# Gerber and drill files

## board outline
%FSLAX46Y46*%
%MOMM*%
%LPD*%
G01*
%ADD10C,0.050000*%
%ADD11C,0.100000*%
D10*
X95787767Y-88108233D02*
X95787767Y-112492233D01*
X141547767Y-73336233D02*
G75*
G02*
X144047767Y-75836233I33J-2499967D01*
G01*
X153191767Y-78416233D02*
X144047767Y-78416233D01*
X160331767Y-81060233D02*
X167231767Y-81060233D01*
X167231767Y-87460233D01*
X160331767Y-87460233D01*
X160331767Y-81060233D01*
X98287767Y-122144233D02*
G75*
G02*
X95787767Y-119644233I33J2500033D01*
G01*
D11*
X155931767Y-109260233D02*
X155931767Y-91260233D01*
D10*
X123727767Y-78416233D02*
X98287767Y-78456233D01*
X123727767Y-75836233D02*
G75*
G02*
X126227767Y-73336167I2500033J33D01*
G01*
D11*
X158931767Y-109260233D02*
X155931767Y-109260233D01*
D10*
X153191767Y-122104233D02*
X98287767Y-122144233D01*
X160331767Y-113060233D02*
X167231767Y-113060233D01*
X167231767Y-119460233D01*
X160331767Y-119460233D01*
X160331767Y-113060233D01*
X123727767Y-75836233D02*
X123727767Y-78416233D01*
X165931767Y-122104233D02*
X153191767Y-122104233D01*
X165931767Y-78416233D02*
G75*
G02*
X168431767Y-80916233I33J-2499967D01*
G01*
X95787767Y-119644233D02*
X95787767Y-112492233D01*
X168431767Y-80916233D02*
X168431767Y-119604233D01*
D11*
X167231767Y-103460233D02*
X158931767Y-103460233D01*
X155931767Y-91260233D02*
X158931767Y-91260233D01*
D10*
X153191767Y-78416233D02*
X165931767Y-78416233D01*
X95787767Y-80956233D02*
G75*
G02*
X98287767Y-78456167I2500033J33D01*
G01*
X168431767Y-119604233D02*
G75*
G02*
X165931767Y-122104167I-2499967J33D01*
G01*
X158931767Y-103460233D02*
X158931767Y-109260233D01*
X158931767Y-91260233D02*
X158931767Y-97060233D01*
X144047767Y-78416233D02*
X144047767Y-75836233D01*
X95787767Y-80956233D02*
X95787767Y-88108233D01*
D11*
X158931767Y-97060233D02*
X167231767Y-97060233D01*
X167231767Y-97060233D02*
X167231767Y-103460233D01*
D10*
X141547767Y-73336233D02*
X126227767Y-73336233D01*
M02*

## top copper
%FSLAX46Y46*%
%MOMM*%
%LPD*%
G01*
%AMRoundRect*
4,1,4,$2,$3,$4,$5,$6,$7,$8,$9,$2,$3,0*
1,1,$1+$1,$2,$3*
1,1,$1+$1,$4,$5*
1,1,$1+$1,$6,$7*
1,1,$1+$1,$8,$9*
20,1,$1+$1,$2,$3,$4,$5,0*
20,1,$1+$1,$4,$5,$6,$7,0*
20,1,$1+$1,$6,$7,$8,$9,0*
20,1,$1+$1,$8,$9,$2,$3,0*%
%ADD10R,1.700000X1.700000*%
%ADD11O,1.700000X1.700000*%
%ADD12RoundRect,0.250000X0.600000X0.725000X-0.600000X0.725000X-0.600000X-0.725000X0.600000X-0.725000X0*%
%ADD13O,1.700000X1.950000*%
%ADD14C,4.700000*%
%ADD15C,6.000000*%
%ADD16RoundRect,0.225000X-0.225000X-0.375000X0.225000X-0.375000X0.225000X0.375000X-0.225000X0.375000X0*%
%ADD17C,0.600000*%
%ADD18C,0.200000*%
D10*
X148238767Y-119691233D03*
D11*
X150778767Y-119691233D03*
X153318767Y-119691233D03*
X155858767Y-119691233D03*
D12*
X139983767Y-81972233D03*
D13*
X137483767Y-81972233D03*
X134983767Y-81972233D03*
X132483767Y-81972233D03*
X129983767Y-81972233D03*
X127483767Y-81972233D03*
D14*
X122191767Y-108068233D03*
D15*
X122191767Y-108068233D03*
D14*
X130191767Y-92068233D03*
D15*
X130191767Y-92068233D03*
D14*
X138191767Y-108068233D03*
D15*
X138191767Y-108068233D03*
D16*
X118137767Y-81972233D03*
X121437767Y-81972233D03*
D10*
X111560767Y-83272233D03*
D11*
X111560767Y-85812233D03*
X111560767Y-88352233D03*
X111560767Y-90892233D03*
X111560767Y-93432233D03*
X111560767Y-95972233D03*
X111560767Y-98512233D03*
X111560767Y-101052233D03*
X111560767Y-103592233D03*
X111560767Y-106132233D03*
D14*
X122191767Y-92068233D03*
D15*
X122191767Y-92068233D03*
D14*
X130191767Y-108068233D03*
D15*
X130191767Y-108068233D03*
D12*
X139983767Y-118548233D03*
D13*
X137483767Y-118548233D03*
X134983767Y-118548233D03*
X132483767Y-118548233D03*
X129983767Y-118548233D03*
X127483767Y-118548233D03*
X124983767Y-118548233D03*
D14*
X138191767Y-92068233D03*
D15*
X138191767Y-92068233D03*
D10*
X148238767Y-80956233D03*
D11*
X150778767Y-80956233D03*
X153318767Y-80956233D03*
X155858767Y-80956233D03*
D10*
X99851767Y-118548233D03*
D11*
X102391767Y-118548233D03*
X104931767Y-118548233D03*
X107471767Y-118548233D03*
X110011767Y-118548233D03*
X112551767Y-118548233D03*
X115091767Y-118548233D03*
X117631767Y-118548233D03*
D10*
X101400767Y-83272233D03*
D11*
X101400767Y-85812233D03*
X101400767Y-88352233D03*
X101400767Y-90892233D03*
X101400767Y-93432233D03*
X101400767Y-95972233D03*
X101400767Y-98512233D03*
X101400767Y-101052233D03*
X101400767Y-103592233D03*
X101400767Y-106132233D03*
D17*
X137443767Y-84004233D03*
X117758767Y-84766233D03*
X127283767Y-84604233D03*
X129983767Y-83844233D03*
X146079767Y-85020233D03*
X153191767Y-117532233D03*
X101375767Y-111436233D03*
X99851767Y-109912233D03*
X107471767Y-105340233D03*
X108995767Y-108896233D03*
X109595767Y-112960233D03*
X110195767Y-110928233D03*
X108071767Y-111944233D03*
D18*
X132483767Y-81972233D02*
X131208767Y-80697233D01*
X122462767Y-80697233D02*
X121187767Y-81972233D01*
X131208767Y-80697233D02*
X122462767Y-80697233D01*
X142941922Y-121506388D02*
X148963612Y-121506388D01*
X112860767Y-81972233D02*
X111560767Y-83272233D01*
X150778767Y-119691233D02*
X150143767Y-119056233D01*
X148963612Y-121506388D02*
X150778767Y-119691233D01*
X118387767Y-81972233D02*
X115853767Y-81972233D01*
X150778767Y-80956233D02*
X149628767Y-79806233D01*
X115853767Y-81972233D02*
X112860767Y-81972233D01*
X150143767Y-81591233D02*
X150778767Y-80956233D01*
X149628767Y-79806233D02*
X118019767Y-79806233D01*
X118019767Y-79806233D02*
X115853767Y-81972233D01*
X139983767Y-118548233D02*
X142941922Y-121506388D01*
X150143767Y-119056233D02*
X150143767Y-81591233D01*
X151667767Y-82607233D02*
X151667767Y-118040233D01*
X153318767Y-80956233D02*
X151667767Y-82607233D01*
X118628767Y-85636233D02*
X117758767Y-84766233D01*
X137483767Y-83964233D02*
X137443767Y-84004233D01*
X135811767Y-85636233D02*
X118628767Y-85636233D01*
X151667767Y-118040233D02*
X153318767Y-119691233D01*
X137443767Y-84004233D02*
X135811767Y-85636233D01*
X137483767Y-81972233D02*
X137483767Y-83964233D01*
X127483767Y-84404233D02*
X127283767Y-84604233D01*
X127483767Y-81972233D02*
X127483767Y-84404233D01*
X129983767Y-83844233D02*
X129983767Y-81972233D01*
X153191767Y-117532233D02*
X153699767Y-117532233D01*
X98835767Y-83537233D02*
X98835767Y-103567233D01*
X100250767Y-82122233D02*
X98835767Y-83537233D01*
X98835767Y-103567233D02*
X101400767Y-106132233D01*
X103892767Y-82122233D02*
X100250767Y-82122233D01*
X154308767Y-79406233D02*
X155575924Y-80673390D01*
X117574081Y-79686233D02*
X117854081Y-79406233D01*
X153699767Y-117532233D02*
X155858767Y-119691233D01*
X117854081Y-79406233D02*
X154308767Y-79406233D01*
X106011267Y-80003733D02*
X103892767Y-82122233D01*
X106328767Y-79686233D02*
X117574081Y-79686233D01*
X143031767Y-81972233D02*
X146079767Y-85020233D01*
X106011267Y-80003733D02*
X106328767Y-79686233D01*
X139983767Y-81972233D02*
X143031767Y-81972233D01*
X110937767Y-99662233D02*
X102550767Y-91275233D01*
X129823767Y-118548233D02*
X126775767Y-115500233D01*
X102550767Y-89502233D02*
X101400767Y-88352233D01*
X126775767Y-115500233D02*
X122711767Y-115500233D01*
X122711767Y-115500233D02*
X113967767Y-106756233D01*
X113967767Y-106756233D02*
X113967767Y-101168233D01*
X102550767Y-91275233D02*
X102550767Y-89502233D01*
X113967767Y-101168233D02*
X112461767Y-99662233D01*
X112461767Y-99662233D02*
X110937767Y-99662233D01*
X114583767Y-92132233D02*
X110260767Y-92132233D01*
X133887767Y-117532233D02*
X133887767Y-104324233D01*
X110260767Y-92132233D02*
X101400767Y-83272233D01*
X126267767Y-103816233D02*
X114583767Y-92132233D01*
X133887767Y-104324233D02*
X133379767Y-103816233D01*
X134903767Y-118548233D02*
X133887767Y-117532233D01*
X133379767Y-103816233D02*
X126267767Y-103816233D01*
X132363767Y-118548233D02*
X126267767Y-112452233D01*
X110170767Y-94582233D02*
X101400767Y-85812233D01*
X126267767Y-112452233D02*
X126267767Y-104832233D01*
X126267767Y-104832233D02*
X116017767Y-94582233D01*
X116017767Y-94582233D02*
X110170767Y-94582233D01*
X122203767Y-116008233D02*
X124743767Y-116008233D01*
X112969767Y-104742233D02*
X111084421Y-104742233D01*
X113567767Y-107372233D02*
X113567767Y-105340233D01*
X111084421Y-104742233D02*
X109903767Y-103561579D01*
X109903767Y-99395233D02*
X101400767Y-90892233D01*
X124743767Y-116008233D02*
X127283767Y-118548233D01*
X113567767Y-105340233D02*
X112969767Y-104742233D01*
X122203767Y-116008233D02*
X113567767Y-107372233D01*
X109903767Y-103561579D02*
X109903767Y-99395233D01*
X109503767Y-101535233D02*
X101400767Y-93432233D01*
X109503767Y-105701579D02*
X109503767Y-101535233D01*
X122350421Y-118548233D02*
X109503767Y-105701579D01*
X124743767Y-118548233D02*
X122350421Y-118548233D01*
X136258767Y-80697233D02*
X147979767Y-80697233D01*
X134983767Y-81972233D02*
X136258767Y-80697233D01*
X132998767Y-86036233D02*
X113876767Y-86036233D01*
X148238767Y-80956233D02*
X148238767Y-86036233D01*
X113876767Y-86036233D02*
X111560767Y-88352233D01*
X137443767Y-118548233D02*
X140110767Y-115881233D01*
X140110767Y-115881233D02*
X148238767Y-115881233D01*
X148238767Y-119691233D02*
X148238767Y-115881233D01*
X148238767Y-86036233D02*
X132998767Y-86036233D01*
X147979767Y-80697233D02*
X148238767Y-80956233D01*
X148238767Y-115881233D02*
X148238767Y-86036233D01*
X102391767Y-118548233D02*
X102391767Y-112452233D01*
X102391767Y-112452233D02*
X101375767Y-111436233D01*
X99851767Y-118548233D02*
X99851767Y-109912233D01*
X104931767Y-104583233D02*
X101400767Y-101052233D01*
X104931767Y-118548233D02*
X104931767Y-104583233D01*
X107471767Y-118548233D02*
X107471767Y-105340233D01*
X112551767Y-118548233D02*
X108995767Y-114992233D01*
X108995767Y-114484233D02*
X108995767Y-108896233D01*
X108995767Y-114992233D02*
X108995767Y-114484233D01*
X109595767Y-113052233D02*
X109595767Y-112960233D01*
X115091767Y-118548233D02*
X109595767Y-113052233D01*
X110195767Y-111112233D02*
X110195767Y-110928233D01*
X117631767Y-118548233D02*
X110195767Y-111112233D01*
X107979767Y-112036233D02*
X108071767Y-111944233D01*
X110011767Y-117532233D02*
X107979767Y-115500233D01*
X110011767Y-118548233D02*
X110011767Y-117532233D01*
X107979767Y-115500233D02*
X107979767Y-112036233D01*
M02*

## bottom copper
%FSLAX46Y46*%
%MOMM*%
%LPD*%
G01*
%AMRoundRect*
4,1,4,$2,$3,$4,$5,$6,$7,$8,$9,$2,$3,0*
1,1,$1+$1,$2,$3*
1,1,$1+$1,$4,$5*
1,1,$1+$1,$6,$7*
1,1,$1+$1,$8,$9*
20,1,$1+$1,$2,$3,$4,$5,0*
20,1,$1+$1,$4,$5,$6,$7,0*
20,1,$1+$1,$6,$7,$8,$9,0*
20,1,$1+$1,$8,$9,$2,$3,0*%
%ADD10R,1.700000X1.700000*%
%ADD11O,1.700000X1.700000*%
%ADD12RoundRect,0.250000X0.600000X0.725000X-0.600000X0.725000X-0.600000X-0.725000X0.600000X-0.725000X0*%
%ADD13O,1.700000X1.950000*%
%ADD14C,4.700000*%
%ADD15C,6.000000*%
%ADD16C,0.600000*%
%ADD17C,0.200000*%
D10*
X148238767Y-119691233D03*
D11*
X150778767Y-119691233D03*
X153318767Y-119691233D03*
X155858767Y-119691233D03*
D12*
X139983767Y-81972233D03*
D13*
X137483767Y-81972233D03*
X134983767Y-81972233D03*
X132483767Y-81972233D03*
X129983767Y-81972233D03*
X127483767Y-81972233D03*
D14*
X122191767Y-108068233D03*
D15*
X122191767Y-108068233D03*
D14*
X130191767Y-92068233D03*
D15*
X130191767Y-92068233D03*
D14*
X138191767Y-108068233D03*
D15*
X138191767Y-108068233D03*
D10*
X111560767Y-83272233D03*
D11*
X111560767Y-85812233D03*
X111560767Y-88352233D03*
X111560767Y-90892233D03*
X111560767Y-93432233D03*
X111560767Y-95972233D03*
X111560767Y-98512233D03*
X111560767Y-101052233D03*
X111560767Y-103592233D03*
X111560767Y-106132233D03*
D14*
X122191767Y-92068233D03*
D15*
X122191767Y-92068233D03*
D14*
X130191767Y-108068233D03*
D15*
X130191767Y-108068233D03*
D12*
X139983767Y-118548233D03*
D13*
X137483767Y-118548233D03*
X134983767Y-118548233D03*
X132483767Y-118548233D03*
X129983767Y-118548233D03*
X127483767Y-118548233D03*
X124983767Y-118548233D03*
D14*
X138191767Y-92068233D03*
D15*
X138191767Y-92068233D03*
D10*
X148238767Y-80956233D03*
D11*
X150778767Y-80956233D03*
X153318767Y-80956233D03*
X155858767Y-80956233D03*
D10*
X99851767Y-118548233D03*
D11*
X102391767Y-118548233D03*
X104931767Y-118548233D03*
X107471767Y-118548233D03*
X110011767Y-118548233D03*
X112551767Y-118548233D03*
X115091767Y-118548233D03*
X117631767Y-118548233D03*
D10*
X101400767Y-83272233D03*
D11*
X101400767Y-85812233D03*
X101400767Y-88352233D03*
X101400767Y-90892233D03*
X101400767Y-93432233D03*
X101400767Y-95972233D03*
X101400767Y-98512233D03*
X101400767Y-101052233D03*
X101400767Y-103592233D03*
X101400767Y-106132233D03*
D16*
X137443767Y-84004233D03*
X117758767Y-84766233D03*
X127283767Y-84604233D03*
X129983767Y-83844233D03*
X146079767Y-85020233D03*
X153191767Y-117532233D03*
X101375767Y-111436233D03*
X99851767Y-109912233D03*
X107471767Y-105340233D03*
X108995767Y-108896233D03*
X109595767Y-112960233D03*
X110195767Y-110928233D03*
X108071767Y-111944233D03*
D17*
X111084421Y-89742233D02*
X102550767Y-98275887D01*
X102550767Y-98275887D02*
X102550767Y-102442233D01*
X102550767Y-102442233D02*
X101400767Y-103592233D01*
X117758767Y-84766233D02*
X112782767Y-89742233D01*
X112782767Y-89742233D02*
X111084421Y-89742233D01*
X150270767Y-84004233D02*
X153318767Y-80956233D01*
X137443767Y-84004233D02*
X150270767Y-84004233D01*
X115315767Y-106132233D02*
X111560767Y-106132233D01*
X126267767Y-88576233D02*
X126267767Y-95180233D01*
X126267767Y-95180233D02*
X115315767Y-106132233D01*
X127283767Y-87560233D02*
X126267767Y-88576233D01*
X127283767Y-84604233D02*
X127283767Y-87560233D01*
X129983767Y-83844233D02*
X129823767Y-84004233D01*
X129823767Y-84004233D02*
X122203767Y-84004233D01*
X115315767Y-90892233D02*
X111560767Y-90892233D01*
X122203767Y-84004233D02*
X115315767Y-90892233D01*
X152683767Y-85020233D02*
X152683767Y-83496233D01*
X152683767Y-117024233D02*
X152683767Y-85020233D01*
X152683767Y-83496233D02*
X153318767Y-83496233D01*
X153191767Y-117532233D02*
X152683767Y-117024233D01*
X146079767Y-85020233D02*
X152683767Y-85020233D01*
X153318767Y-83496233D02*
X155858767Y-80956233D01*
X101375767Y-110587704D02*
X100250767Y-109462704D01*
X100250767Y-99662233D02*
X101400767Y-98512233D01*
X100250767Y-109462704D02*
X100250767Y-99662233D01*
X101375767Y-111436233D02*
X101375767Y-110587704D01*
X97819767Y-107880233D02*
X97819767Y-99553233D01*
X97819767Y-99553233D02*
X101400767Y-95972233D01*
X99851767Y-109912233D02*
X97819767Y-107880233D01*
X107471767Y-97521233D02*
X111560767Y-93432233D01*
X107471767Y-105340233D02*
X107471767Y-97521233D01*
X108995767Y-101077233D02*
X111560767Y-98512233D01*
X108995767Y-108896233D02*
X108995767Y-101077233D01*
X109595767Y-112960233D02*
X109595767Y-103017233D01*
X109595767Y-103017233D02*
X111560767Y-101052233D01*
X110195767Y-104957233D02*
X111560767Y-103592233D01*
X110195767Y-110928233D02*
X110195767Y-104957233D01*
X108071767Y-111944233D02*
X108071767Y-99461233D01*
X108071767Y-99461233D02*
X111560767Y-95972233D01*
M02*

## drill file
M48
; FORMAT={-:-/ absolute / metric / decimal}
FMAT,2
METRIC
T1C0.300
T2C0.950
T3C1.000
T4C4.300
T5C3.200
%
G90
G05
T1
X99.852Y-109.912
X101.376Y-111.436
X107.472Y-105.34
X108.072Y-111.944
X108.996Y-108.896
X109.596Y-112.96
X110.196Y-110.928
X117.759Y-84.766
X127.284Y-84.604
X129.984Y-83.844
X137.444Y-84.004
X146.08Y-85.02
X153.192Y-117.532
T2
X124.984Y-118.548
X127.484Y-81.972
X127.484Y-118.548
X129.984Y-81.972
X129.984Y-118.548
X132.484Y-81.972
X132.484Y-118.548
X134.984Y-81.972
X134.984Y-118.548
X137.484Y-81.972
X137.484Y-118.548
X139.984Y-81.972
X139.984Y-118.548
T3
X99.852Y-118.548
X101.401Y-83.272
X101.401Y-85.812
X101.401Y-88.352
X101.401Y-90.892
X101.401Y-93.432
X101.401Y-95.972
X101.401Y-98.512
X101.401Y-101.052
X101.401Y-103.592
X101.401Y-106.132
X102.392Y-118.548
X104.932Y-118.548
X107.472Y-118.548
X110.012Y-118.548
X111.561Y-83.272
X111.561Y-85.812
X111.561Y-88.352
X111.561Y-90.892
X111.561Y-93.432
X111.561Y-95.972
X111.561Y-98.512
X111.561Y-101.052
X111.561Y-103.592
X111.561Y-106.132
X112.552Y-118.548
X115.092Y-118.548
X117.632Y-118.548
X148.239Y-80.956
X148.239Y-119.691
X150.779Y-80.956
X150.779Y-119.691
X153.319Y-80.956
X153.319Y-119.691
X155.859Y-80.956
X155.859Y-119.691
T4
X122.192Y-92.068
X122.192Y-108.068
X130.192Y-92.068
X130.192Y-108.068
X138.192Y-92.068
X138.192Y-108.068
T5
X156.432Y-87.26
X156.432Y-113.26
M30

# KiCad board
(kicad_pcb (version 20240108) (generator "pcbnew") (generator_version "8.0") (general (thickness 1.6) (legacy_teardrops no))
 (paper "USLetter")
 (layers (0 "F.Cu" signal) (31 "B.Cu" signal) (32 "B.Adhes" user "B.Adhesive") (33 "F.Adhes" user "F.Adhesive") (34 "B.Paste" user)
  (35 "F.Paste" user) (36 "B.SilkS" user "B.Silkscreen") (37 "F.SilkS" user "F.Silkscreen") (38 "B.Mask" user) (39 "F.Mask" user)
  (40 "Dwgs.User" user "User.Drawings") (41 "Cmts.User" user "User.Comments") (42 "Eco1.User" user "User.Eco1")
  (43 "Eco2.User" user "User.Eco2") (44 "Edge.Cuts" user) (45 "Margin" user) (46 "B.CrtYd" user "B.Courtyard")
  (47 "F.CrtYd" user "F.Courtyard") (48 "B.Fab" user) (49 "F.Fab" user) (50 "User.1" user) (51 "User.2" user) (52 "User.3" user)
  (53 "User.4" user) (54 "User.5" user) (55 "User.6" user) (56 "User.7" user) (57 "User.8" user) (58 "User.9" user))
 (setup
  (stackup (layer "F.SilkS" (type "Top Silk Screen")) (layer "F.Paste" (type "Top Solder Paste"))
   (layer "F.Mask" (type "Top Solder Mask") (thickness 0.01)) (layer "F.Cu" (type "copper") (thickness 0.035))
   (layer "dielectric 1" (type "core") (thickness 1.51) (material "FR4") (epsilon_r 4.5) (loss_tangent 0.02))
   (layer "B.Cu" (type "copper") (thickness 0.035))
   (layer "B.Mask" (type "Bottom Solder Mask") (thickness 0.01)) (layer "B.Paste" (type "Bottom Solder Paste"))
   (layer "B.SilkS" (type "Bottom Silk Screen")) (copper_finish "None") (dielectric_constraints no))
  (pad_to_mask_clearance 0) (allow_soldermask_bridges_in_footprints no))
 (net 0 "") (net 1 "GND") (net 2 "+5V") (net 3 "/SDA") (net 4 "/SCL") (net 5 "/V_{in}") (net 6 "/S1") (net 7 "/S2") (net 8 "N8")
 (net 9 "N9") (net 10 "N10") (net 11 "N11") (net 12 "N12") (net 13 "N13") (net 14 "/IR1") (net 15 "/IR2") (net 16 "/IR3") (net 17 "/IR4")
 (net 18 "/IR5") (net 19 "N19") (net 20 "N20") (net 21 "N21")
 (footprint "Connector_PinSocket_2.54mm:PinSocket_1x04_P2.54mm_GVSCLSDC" (layer "F.Cu") (at 148.238767 119.691233 90)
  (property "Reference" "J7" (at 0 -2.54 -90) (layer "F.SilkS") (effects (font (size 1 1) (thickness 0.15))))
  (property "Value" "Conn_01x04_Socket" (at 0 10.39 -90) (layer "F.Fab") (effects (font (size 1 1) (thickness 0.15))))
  (pad "1" thru_hole rect (at 0 0 90) (size 1.7 1.7) (drill 1) (layers "*.Cu" "*.Mask") (remove_unused_layers no) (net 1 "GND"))
  (pad "2" thru_hole oval (at 0 2.54 90) (size 1.7 1.7) (drill 1) (layers "*.Cu" "*.Mask") (remove_unused_layers no) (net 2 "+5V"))
  (pad "3" thru_hole oval (at 0 5.08 90) (size 1.7 1.7) (drill 1) (layers "*.Cu" "*.Mask") (remove_unused_layers no) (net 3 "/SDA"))
  (pad "4" thru_hole oval (at 0 7.62 90) (size 1.7 1.7) (drill 1) (layers "*.Cu" "*.Mask") (remove_unused_layers no) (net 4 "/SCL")))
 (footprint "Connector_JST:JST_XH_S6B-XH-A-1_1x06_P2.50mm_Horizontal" (layer "F.Cu") (at 139.983767 81.972233 180)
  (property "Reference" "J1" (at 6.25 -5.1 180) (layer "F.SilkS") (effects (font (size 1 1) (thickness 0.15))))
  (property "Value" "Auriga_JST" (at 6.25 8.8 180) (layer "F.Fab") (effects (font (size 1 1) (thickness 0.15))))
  (pad "1" thru_hole roundrect (at 0 0 180) (size 1.7 1.95) (drill 0.95) (layers "*.Cu" "*.Mask") (remove_unused_layers no)
   (roundrect_rratio 0.147059) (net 4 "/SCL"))
  (pad "2" thru_hole oval (at 2.5 0 180) (size 1.7 1.95) (drill 0.95) (layers "*.Cu" "*.Mask") (remove_unused_layers no) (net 3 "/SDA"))
  (pad "3" thru_hole oval (at 5 0 180) (size 1.7 1.95) (drill 0.95) (layers "*.Cu" "*.Mask") (remove_unused_layers no) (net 1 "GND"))
  (pad "4" thru_hole oval (at 7.5 0 180) (size 1.7 1.95) (drill 0.95) (layers "*.Cu" "*.Mask") (remove_unused_layers no) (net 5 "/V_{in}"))
  (pad "5" thru_hole oval (at 10 0 180) (size 1.7 1.95) (drill 0.95) (layers "*.Cu" "*.Mask") (remove_unused_layers no) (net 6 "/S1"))
  (pad "6" thru_hole oval (at 12.5 0 180) (size 1.7 1.95) (drill 0.95) (layers "*.Cu" "*.Mask") (remove_unused_layers no) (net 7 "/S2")))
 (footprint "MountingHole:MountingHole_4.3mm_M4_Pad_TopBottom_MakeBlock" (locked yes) (layer "F.Cu") (at 122.191767 108.068233)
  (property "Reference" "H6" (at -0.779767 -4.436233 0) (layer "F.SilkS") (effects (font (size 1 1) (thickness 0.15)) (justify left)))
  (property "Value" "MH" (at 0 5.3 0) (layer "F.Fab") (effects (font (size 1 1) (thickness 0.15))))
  (pad "1" thru_hole circle (at 0 0) (size 4.7 4.7) (drill 4.3) (layers "*.Cu" "*.Mask") (remove_unused_layers no))
  (pad "1" connect circle (at 0 0) (size 6 6) (layers "F.Cu" "F.Mask"))
  (pad "1" connect circle (at 0 0) (size 6 6) (layers "B.Cu" "B.Mask")))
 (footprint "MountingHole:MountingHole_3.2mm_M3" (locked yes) (layer "F.Cu") (at 156.431767 113.260233)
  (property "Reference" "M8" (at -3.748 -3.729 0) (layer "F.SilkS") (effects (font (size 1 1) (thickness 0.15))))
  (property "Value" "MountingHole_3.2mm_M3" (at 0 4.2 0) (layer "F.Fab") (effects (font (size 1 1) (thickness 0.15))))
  (pad "" np_thru_hole circle (at 0 0) (size 3.2 3.2) (drill 3.2) (layers "*.Cu" "*.Mask")))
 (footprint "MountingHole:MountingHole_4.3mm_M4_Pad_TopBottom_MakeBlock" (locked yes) (layer "F.Cu") (at 130.191767 92.068233)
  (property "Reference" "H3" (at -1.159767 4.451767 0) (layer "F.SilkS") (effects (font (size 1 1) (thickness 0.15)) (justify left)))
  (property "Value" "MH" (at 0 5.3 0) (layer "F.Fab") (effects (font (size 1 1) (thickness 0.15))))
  (pad "1" thru_hole circle (at 0 0) (size 4.7 4.7) (drill 4.3) (layers "*.Cu" "*.Mask") (remove_unused_layers no))
  (pad "1" connect circle (at 0 0) (size 6 6) (layers "F.Cu" "F.Mask"))
  (pad "1" connect circle (at 0 0) (size 6 6) (layers "B.Cu" "B.Mask")))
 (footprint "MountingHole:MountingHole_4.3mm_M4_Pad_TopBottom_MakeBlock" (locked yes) (layer "F.Cu") (at 138.191767 108.068233)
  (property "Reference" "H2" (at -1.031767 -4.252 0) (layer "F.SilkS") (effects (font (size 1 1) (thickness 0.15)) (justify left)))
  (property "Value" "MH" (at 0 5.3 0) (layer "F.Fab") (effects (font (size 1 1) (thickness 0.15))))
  (pad "1" thru_hole circle (at 0 0) (size 4.7 4.7) (drill 4.3) (layers "*.Cu" "*.Mask") (remove_unused_layers no))
  (pad "1" connect circle (at 0 0) (size 6 6) (layers "F.Cu" "F.Mask"))
  (pad "1" connect circle (at 0 0) (size 6 6) (layers "B.Cu" "B.Mask")))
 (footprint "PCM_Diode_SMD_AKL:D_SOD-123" (layer "F.Cu") (at 119.787767 81.972233)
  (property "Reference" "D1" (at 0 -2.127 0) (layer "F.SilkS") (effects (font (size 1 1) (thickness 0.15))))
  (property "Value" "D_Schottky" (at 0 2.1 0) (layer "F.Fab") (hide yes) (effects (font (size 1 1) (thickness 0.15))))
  (pad "1" smd roundrect (at -1.65 0) (size 0.9 1.2) (layers "F.Cu" "F.Paste" "F.Mask") (roundrect_rratio 0.25) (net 2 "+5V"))
  (pad "2" smd roundrect (at 1.65 0) (size 0.9 1.2) (layers "F.Cu" "F.Paste" "F.Mask") (roundrect_rratio 0.25) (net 5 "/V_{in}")))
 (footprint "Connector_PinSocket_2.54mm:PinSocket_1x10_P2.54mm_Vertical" (layer "F.Cu") (at 111.560767 83.272233)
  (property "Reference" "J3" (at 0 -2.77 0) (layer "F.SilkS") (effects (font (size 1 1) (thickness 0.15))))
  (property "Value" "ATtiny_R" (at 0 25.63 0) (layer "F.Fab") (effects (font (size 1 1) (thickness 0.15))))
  (pad "1" thru_hole rect (at 0 0) (size 1.7 1.7) (drill 1) (layers "*.Cu" "*.Mask") (remove_unused_layers no) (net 2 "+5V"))
  (pad "2" thru_hole oval (at 0 2.54) (size 1.7 1.7) (drill 1) (layers "*.Cu" "*.Mask") (remove_unused_layers no) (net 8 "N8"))
  (pad "3" thru_hole oval (at 0 5.08) (size 1.7 1.7) (drill 1) (layers "*.Cu" "*.Mask") (remove_unused_layers no) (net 1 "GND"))
  (pad "4" thru_hole oval (at 0 7.62) (size 1.7 1.7) (drill 1) (layers "*.Cu" "*.Mask") (remove_unused_layers no) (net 6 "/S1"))
  (pad "5" thru_hole oval (at 0 10.16) (size 1.7 1.7) (drill 1) (layers "*.Cu" "*.Mask") (remove_unused_layers no) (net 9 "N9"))
  (pad "6" thru_hole oval (at 0 12.7) (size 1.7 1.7) (drill 1) (layers "*.Cu" "*.Mask") (remove_unused_layers no) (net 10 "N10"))
  (pad "7" thru_hole oval (at 0 15.24) (size 1.7 1.7) (drill 1) (layers "*.Cu" "*.Mask") (remove_unused_layers no) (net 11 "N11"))
  (pad "8" thru_hole oval (at 0 17.78) (size 1.7 1.7) (drill 1) (layers "*.Cu" "*.Mask") (remove_unused_layers no) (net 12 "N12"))
  (pad "9" thru_hole oval (at 0 20.32) (size 1.7 1.7) (drill 1) (layers "*.Cu" "*.Mask") (remove_unused_layers no) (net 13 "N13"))
  (pad "10" thru_hole oval (at 0 22.86) (size 1.7 1.7) (drill 1) (layers "*.Cu" "*.Mask") (remove_unused_layers no) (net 7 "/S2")))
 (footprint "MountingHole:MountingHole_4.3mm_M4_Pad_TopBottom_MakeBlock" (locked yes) (layer "F.Cu") (at 122.191767 92.068233)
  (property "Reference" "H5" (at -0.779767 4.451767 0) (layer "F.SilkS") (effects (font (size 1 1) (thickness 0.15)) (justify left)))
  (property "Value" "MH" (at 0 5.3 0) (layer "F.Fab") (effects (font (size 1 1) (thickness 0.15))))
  (pad "1" thru_hole circle (at 0 0) (size 4.7 4.7) (drill 4.3) (layers "*.Cu" "*.Mask") (remove_unused_layers no))
  (pad "1" connect circle (at 0 0) (size 6 6) (layers "F.Cu" "F.Mask"))
  (pad "1" connect circle (at 0 0) (size 6 6) (layers "B.Cu" "B.Mask")))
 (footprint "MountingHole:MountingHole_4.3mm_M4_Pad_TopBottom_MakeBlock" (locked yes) (layer "F.Cu") (at 130.191767 108.068233)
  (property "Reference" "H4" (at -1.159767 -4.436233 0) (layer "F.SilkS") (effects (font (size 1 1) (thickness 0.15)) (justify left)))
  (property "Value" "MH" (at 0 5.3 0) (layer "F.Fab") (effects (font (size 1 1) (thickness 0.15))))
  (pad "1" thru_hole circle (at 0 0) (size 4.7 4.7) (drill 4.3) (layers "*.Cu" "*.Mask") (remove_unused_layers no))
  (pad "1" connect circle (at 0 0) (size 6 6) (layers "F.Cu" "F.Mask"))
  (pad "1" connect circle (at 0 0) (size 6 6) (layers "B.Cu" "B.Mask")))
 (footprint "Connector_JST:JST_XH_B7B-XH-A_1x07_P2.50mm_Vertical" (layer "F.Cu") (at 139.983767 118.548233 180)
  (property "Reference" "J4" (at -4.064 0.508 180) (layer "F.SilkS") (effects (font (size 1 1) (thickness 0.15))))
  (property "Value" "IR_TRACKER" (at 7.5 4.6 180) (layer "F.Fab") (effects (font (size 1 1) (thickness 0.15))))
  (pad "1" thru_hole roundrect (at 0 0 180) (size 1.7 1.95) (drill 0.95) (layers "*.Cu" "*.Mask") (remove_unused_layers no)
   (roundrect_rratio 0.147059) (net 2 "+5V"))
  (pad "2" thru_hole oval (at 2.5 0 180) (size 1.7 1.95) (drill 0.95) (layers "*.Cu" "*.Mask") (remove_unused_layers no) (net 1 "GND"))
  (pad "3" thru_hole oval (at 5 0 180) (size 1.7 1.95) (drill 0.95) (layers "*.Cu" "*.Mask") (remove_unused_layers no) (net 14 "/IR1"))
  (pad "4" thru_hole oval (at 7.5 0 180) (size 1.7 1.95) (drill 0.95) (layers "*.Cu" "*.Mask") (remove_unused_layers no) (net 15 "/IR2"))
  (pad "5" thru_hole oval (at 10 0 180) (size 1.7 1.95) (drill 0.95) (layers "*.Cu" "*.Mask") (remove_unused_layers no) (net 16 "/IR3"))
  (pad "6" thru_hole oval (at 12.5 0 180) (size 1.7 1.95) (drill 0.95) (layers "*.Cu" "*.Mask") (remove_unused_layers no) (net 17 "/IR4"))
  (pad "7" thru_hole oval (at 15 0 180) (size 1.7 1.95) (drill 0.95) (layers "*.Cu" "*.Mask") (remove_unused_layers no) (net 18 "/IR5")))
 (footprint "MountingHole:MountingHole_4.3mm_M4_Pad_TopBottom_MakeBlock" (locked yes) (layer "F.Cu") (at 138.191767 92.068233)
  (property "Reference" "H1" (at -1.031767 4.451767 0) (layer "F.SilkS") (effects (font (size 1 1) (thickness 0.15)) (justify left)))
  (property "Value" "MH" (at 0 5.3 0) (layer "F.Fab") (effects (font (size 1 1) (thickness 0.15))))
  (pad "1" thru_hole circle (at 0 0) (size 4.7 4.7) (drill 4.3) (layers "*.Cu" "*.Mask") (remove_unused_layers no))
  (pad "1" connect circle (at 0 0) (size 6 6) (layers "F.Cu" "F.Mask"))
  (pad "1" connect circle (at 0 0) (size 6 6) (layers "B.Cu" "B.Mask")))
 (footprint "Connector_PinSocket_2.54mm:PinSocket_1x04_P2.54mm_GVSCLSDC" (layer "F.Cu") (at 148.238767 80.956233 90)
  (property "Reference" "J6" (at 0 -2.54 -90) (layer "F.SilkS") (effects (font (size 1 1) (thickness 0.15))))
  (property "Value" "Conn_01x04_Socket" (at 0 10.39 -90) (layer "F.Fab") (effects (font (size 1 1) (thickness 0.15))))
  (pad "1" thru_hole rect (at 0 0 90) (size 1.7 1.7) (drill 1) (layers "*.Cu" "*.Mask") (remove_unused_layers no) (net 1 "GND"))
  (pad "2" thru_hole oval (at 0 2.54 90) (size 1.7 1.7) (drill 1) (layers "*.Cu" "*.Mask") (remove_unused_layers no) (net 2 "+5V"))
  (pad "3" thru_hole oval (at 0 5.08 90) (size 1.7 1.7) (drill 1) (layers "*.Cu" "*.Mask") (remove_unused_layers no) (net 3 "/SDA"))
  (pad "4" thru_hole oval (at 0 7.62 90) (size 1.7 1.7) (drill 1) (layers "*.Cu" "*.Mask") (remove_unused_layers no) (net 4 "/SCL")))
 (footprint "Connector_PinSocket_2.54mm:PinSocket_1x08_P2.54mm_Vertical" (layer "F.Cu") (at 99.851767 118.548233 90)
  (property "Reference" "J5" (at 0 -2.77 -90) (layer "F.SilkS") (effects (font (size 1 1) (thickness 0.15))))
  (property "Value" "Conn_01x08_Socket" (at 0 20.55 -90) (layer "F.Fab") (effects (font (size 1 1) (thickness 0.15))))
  (pad "1" thru_hole rect (at 0 0 90) (size 1.7 1.7) (drill 1) (layers "*.Cu" "*.Mask") (remove_unused_layers no) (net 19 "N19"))
  (pad "2" thru_hole oval (at 0 2.54 90) (size 1.7 1.7) (drill 1) (layers "*.Cu" "*.Mask") (remove_unused_layers no) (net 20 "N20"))
  (pad "3" thru_hole oval (at 0 5.08 90) (size 1.7 1.7) (drill 1) (layers "*.Cu" "*.Mask") (remove_unused_layers no) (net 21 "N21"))
  (pad "4" thru_hole oval (at 0 7.62 90) (size 1.7 1.7) (drill 1) (layers "*.Cu" "*.Mask") (remove_unused_layers no) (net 9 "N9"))
  (pad "5" thru_hole oval (at 0 10.16 90) (size 1.7 1.7) (drill 1) (layers "*.Cu" "*.Mask") (remove_unused_layers no) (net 10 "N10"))
  (pad "6" thru_hole oval (at 0 12.7 90) (size 1.7 1.7) (drill 1) (layers "*.Cu" "*.Mask") (remove_unused_layers no) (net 11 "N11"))
  (pad "7" thru_hole oval (at 0 15.24 90) (size 1.7 1.7) (drill 1) (layers "*.Cu" "*.Mask") (remove_unused_layers no) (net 12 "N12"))
  (pad "8" thru_hole oval (at 0 17.78 90) (size 1.7 1.7) (drill 1) (layers "*.Cu" "*.Mask") (remove_unused_layers no) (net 13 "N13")))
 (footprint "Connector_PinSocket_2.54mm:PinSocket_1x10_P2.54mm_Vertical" (layer "F.Cu") (at 101.400767 83.272233)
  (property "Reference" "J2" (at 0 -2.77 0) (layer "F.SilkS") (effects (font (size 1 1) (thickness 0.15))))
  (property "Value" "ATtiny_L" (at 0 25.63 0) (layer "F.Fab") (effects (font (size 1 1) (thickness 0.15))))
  (pad "1" thru_hole rect (at 0 0) (size 1.7 1.7) (drill 1) (layers "*.Cu" "*.Mask") (remove_unused_layers no) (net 14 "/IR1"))
  (pad "2" thru_hole oval (at 0 2.54) (size 1.7 1.7) (drill 1) (layers "*.Cu" "*.Mask") (remove_unused_layers no) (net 15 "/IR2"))
  (pad "3" thru_hole oval (at 0 5.08) (size 1.7 1.7) (drill 1) (layers "*.Cu" "*.Mask") (remove_unused_layers no) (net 16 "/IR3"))
  (pad "4" thru_hole oval (at 0 7.62) (size 1.7 1.7) (drill 1) (layers "*.Cu" "*.Mask") (remove_unused_layers no) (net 17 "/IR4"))
  (pad "5" thru_hole oval (at 0 10.16) (size 1.7 1.7) (drill 1) (layers "*.Cu" "*.Mask") (remove_unused_layers no) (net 18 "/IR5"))
  (pad "6" thru_hole oval (at 0 12.7) (size 1.7 1.7) (drill 1) (layers "*.Cu" "*.Mask") (remove_unused_layers no) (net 19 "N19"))
  (pad "7" thru_hole oval (at 0 15.24) (size 1.7 1.7) (drill 1) (layers "*.Cu" "*.Mask") (remove_unused_layers no) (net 20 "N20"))
  (pad "8" thru_hole oval (at 0 17.78) (size 1.7 1.7) (drill 1) (layers "*.Cu" "*.Mask") (remove_unused_layers no) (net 21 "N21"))
  (pad "9" thru_hole oval (at 0 20.32) (size 1.7 1.7) (drill 1) (layers "*.Cu" "*.Mask") (remove_unused_layers no) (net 3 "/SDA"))
  (pad "10" thru_hole oval (at 0 22.86) (size 1.7 1.7) (drill 1) (layers "*.Cu" "*.Mask") (remove_unused_layers no) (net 4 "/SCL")))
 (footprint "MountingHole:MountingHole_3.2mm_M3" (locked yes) (layer "F.Cu") (at 156.431767 87.260233)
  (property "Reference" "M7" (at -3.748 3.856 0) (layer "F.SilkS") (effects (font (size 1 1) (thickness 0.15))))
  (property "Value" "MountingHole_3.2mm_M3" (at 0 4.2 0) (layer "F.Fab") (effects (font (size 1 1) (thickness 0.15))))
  (pad "" np_thru_hole circle (at 0 0) (size 3.2 3.2) (drill 3.2) (layers "*.Cu" "*.Mask")))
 (gr_line (start 95.787767 88.108233) (end 95.787767 112.492233) (stroke (width 0.05) (type default)) (layer "Edge.Cuts"))
 (gr_arc (start 141.547767 73.336233) (mid 143.315534 74.068466) (end 144.047767 75.836233) (stroke (width 0.05) (type default))
  (layer "Edge.Cuts"))
 (gr_line (start 153.191767 78.416233) (end 144.047767 78.416233) (stroke (width 0.05) (type default)) (layer "Edge.Cuts"))
 (gr_rect (start 160.331767 81.060233) (end 167.231767 87.460233) (locked yes) (stroke (width 0.05) (type default)) (fill none)
  (layer "Edge.Cuts"))
 (gr_arc (start 98.287767 122.144233) (mid 96.52 121.412) (end 95.787767 119.644233) (stroke (width 0.05) (type default))
  (layer "Edge.Cuts"))
 (gr_line (start 155.931767 109.260233) (end 155.931767 91.260233) (locked yes) (stroke (width 0.1) (type default)) (layer "Edge.Cuts"))
 (gr_line (start 123.727767 78.416233) (end 98.287767 78.456233) (stroke (width 0.05) (type default)) (layer "Edge.Cuts"))
 (gr_arc (start 123.727767 75.836233) (mid 124.46 74.068466) (end 126.227767 73.336233) (stroke (width 0.05) (type default))
  (layer "Edge.Cuts"))
 (gr_line (start 158.931767 109.260233) (end 155.931767 109.260233) (locked yes) (stroke (width 0.1) (type default)) (layer "Edge.Cuts"))
 (gr_line (start 153.191767 122.104233) (end 98.287767 122.144233) (stroke (width 0.05) (type default)) (layer "Edge.Cuts"))
 (gr_rect (start 160.331767 113.060233) (end 167.231767 119.460233) (locked yes) (stroke (width 0.05) (type default)) (fill none)
  (layer "Edge.Cuts"))
 (gr_line (start 123.727767 75.836233) (end 123.727767 78.416233) (stroke (width 0.05) (type default)) (layer "Edge.Cuts"))
 (gr_line (start 165.931767 122.104233) (end 153.191767 122.104233) (stroke (width 0.05) (type default)) (layer "Edge.Cuts"))
 (gr_arc (start 165.931767 78.416233) (mid 167.699534 79.148466) (end 168.431767 80.916233) (locked yes)
  (stroke (width 0.05) (type default)) (layer "Edge.Cuts"))
 (gr_line (start 95.787767 119.644233) (end 95.787767 112.492233) (stroke (width 0.05) (type default)) (layer "Edge.Cuts"))
 (gr_line (start 168.431767 80.916233) (end 168.431767 119.604233) (locked yes) (stroke (width 0.05) (type default)) (layer "Edge.Cuts"))
 (gr_line (start 167.231767 103.460233) (end 158.931767 103.460233) (locked yes) (stroke (width 0.1) (type default)) (layer "Edge.Cuts"))
 (gr_line (start 155.931767 91.260233) (end 158.931767 91.260233) (locked yes) (stroke (width 0.1) (type default)) (layer "Edge.Cuts"))
 (gr_line (start 153.191767 78.416233) (end 165.931767 78.416233) (stroke (width 0.05) (type default)) (layer "Edge.Cuts"))
 (gr_arc (start 95.787767 80.956233) (mid 96.52 79.188466) (end 98.287767 78.456233) (stroke (width 0.05) (type default))
  (layer "Edge.Cuts"))
 (gr_arc (start 168.431767 119.604233) (mid 167.699534 121.372) (end 165.931767 122.104233) (locked yes)
  (stroke (width 0.05) (type default)) (layer "Edge.Cuts"))
 (gr_line (start 158.931767 103.460233) (end 158.931767 109.260233) (locked yes) (stroke (width 0.05) (type default)) (layer "Edge.Cuts"))
 (gr_line (start 158.931767 91.260233) (end 158.931767 97.060233) (locked yes) (stroke (width 0.05) (type default)) (layer "Edge.Cuts"))
 (gr_line (start 144.047767 78.416233) (end 144.047767 75.836233) (stroke (width 0.05) (type default)) (layer "Edge.Cuts"))
 (gr_line (start 95.787767 80.956233) (end 95.787767 88.108233) (stroke (width 0.05) (type default)) (layer "Edge.Cuts"))
 (gr_line (start 158.931767 97.060233) (end 167.231767 97.060233) (locked yes) (stroke (width 0.1) (type default)) (layer "Edge.Cuts"))
 (gr_line (start 167.231767 97.060233) (end 167.231767 103.460233) (locked yes) (stroke (width 0.1) (type default)) (layer "Edge.Cuts"))
 (gr_line (start 141.547767 73.336233) (end 126.227767 73.336233) (stroke (width 0.05) (type default)) (layer "Edge.Cuts"))
 (segment (start 132.483767 81.972233) (end 131.208767 80.697233) (width 0.2) (layer "F.Cu") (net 5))
 (segment (start 122.462767 80.697233) (end 121.187767 81.972233) (width 0.2) (layer "F.Cu") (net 5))
 (segment (start 131.208767 80.697233) (end 122.462767 80.697233) (width 0.2) (layer "F.Cu") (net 5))
 (segment (start 142.941922 121.506388) (end 148.963612 121.506388) (width 0.2) (layer "F.Cu") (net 2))
 (segment (start 112.860767 81.972233) (end 111.560767 83.272233) (width 0.2) (layer "F.Cu") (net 2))
 (segment (start 150.778767 119.691233) (end 150.143767 119.056233) (width 0.2) (layer "F.Cu") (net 2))
 (segment (start 148.963612 121.506388) (end 150.778767 119.691233) (width 0.2) (layer "F.Cu") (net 2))
 (segment (start 118.387767 81.972233) (end 115.853767 81.972233) (width 0.2) (layer "F.Cu") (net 2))
 (segment (start 150.778767 80.956233) (end 149.628767 79.806233) (width 0.2) (layer "F.Cu") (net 2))
 (segment (start 115.853767 81.972233) (end 112.860767 81.972233) (width 0.2) (layer "F.Cu") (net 2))
 (segment (start 150.143767 81.591233) (end 150.778767 80.956233) (width 0.2) (layer "F.Cu") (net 2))
 (segment (start 149.628767 79.806233) (end 118.019767 79.806233) (width 0.2) (layer "F.Cu") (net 2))
 (segment (start 118.019767 79.806233) (end 115.853767 81.972233) (width 0.2) (layer "F.Cu") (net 2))
 (segment (start 139.983767 118.548233) (end 142.941922 121.506388) (width 0.2) (layer "F.Cu") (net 2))
 (segment (start 150.143767 119.056233) (end 150.143767 81.591233) (width 0.2) (layer "F.Cu") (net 2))
 (segment (start 151.667767 82.607233) (end 151.667767 118.040233) (width 0.2) (layer "F.Cu") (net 3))
 (segment (start 153.318767 80.956233) (end 151.667767 82.607233) (width 0.2) (layer "F.Cu") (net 3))
 (segment (start 118.628767 85.636233) (end 117.758767 84.766233) (width 0.2) (layer "F.Cu") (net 3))
 (segment (start 137.483767 83.964233) (end 137.443767 84.004233) (width 0.2) (layer "F.Cu") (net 3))
 (segment (start 135.811767 85.636233) (end 118.628767 85.636233) (width 0.2) (layer "F.Cu") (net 3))
 (segment (start 151.667767 118.040233) (end 153.318767 119.691233) (width 0.2) (layer "F.Cu") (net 3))
 (segment (start 137.443767 84.004233) (end 135.811767 85.636233) (width 0.2) (layer "F.Cu") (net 3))
 (segment (start 137.483767 81.972233) (end 137.483767 83.964233) (width 0.2) (layer "F.Cu") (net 3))
 (via (at 137.443767 84.004233) (size 0.6) (drill 0.3) (layers "F.Cu" "B.Cu") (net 3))
 (via blind (at 117.758767 84.766233) (size 0.6) (drill 0.3) (layers "F.Cu" "B.Cu") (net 3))
 (segment (start 111.084421 89.742233) (end 102.550767 98.275887) (width 0.2) (layer "B.Cu") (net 3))
 (segment (start 102.550767 98.275887) (end 102.550767 102.442233) (width 0.2) (layer "B.Cu") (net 3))
 (segment (start 102.550767 102.442233) (end 101.400767 103.592233) (width 0.2) (layer "B.Cu") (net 3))
 (segment (start 117.758767 84.766233) (end 112.782767 89.742233) (width 0.2) (layer "B.Cu") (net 3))
 (segment (start 112.782767 89.742233) (end 111.084421 89.742233) (width 0.2) (layer "B.Cu") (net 3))
 (segment (start 150.270767 84.004233) (end 153.318767 80.956233) (width 0.2) (layer "B.Cu") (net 3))
 (segment (start 137.443767 84.004233) (end 150.270767 84.004233) (width 0.2) (layer "B.Cu") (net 3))
 (segment (start 127.483767 84.404233) (end 127.283767 84.604233) (width 0.2) (layer "F.Cu") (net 7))
 (segment (start 127.483767 81.972233) (end 127.483767 84.404233) (width 0.2) (layer "F.Cu") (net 7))
 (via (at 127.283767 84.604233) (size 0.6) (drill 0.3) (layers "F.Cu" "B.Cu") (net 7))
 (segment (start 115.315767 106.132233) (end 111.560767 106.132233) (width 0.2) (layer "B.Cu") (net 7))
 (segment (start 126.267767 88.576233) (end 126.267767 95.180233) (width 0.2) (layer "B.Cu") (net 7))
 (segment (start 126.267767 95.180233) (end 115.315767 106.132233) (width 0.2) (layer "B.Cu") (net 7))
 (segment (start 127.283767 87.560233) (end 126.267767 88.576233) (width 0.2) (layer "B.Cu") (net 7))
 (segment (start 127.283767 84.604233) (end 127.283767 87.560233) (width 0.2) (layer "B.Cu") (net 7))
 (segment (start 129.983767 83.844233) (end 129.983767 81.972233) (width 0.2) (layer "F.Cu") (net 6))
 (via blind (at 129.983767 83.844233) (size 0.6) (drill 0.3) (layers "F.Cu" "B.Cu") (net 6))
 (segment (start 129.983767 83.844233) (end 129.823767 84.004233) (width 0.2) (layer "B.Cu") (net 6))
 (segment (start 129.823767 84.004233) (end 122.203767 84.004233) (width 0.2) (layer "B.Cu") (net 6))
 (segment (start 115.315767 90.892233) (end 111.560767 90.892233) (width 0.2) (layer "B.Cu") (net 6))
 (segment (start 122.203767 84.004233) (end 115.315767 90.892233) (width 0.2) (layer "B.Cu") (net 6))
 (segment (start 153.191767 117.532233) (end 153.699767 117.532233) (width 0.2) (layer "F.Cu") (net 4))
 (segment (start 98.835767 83.537233) (end 98.835767 103.567233) (width 0.2) (layer "F.Cu") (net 4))
 (segment (start 100.250767 82.122233) (end 98.835767 83.537233) (width 0.2) (layer "F.Cu") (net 4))
 (segment (start 98.835767 103.567233) (end 101.400767 106.132233) (width 0.2) (layer "F.Cu") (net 4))
 (segment (start 103.892767 82.122233) (end 100.250767 82.122233) (width 0.2) (layer "F.Cu") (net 4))
 (segment (start 154.308767 79.406233) (end 155.575924 80.67339) (width 0.2) (layer "F.Cu") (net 4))
 (segment (start 117.574081 79.686233) (end 117.854081 79.406233) (width 0.2) (layer "F.Cu") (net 4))
 (segment (start 153.699767 117.532233) (end 155.858767 119.691233) (width 0.2) (layer "F.Cu") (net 4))
 (segment (start 117.854081 79.406233) (end 154.308767 79.406233) (width 0.2) (layer "F.Cu") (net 4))
 (segment (start 106.011267 80.003733) (end 103.892767 82.122233) (width 0.2) (layer "F.Cu") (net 4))
 (segment (start 106.328767 79.686233) (end 117.574081 79.686233) (width 0.2) (layer "F.Cu") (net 4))
 (segment (start 143.031767 81.972233) (end 146.079767 85.020233) (width 0.2) (layer "F.Cu") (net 4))
 (segment (start 106.011267 80.003733) (end 106.328767 79.686233) (width 0.2) (layer "F.Cu") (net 4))
 (segment (start 139.983767 81.972233) (end 143.031767 81.972233) (width 0.2) (layer "F.Cu") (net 4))
 (via (at 146.079767 85.020233) (size 0.6) (drill 0.3) (layers "F.Cu" "B.Cu") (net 4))
 (via blind (at 153.191767 117.532233) (size 0.6) (drill 0.3) (layers "F.Cu" "B.Cu") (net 4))
 (segment (start 152.683767 85.020233) (end 152.683767 83.496233) (width 0.2) (layer "B.Cu") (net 4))
 (segment (start 152.683767 117.024233) (end 152.683767 85.020233) (width 0.2) (layer "B.Cu") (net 4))
 (segment (start 152.683767 83.496233) (end 153.318767 83.496233) (width 0.2) (layer "B.Cu") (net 4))
 (segment (start 153.191767 117.532233) (end 152.683767 117.024233) (width 0.2) (layer "B.Cu") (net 4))
 (segment (start 146.079767 85.020233) (end 152.683767 85.020233) (width 0.2) (layer "B.Cu") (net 4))
 (segment (start 153.318767 83.496233) (end 155.858767 80.956233) (width 0.2) (layer "B.Cu") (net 4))
 (segment (start 110.937767 99.662233) (end 102.550767 91.275233) (width 0.2) (layer "F.Cu") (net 16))
 (segment (start 129.823767 118.548233) (end 126.775767 115.500233) (width 0.2) (layer "F.Cu") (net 16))
 (segment (start 102.550767 89.502233) (end 101.400767 88.352233) (width 0.2) (layer "F.Cu") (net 16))
 (segment (start 126.775767 115.500233) (end 122.711767 115.500233) (width 0.2) (layer "F.Cu") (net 16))
 (segment (start 122.711767 115.500233) (end 113.967767 106.756233) (width 0.2) (layer "F.Cu") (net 16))
 (segment (start 113.967767 106.756233) (end 113.967767 101.168233) (width 0.2) (layer "F.Cu") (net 16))
 (segment (start 102.550767 91.275233) (end 102.550767 89.502233) (width 0.2) (layer "F.Cu") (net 16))
 (segment (start 113.967767 101.168233) (end 112.461767 99.662233) (width 0.2) (layer "F.Cu") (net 16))
 (segment (start 112.461767 99.662233) (end 110.937767 99.662233) (width 0.2) (layer "F.Cu") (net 16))
 (segment (start 114.583767 92.132233) (end 110.260767 92.132233) (width 0.2) (layer "F.Cu") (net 14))
 (segment (start 133.887767 117.532233) (end 133.887767 104.324233) (width 0.2) (layer "F.Cu") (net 14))
 (segment (start 110.260767 92.132233) (end 101.400767 83.272233) (width 0.2) (layer "F.Cu") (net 14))
 (segment (start 126.267767 103.816233) (end 114.583767 92.132233) (width 0.2) (layer "F.Cu") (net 14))
 (segment (start 133.887767 104.324233) (end 133.379767 103.816233) (width 0.2) (layer "F.Cu") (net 14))
 (segment (start 134.903767 118.548233) (end 133.887767 117.532233) (width 0.2) (layer "F.Cu") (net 14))
 (segment (start 133.379767 103.816233) (end 126.267767 103.816233) (width 0.2) (layer "F.Cu") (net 14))
 (segment (start 132.363767 118.548233) (end 126.267767 112.452233) (width 0.2) (layer "F.Cu") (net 15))
 (segment (start 110.170767 94.582233) (end 101.400767 85.812233) (width 0.2) (layer "F.Cu") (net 15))
 (segment (start 126.267767 112.452233) (end 126.267767 104.832233) (width 0.2) (layer "F.Cu") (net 15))
 (segment (start 126.267767 104.832233) (end 116.017767 94.582233) (width 0.2) (layer "F.Cu") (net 15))
 (segment (start 116.017767 94.582233) (end 110.170767 94.582233) (width 0.2) (layer "F.Cu") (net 15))
 (segment (start 122.203767 116.008233) (end 124.743767 116.008233) (width 0.2) (layer "F.Cu") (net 17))
 (segment (start 112.969767 104.742233) (end 111.084421 104.742233) (width 0.2) (layer "F.Cu") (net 17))
 (segment (start 113.567767 107.372233) (end 113.567767 105.340233) (width 0.2) (layer "F.Cu") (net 17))
 (segment (start 111.084421 104.742233) (end 109.903767 103.561579) (width 0.2) (layer "F.Cu") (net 17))
 (segment (start 109.903767 99.395233) (end 101.400767 90.892233) (width 0.2) (layer "F.Cu") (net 17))
 (segment (start 124.743767 116.008233) (end 127.283767 118.548233) (width 0.2) (layer "F.Cu") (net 17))
 (segment (start 113.567767 105.340233) (end 112.969767 104.742233) (width 0.2) (layer "F.Cu") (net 17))
 (segment (start 122.203767 116.008233) (end 113.567767 107.372233) (width 0.2) (layer "F.Cu") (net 17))
 (segment (start 109.903767 103.561579) (end 109.903767 99.395233) (width 0.2) (layer "F.Cu") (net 17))
 (segment (start 109.503767 101.535233) (end 101.400767 93.432233) (width 0.2) (layer "F.Cu") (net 18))
 (segment (start 109.503767 105.701579) (end 109.503767 101.535233) (width 0.2) (layer "F.Cu") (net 18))
 (segment (start 122.350421 118.548233) (end 109.503767 105.701579) (width 0.2) (layer "F.Cu") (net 18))
 (segment (start 124.743767 118.548233) (end 122.350421 118.548233) (width 0.2) (layer "F.Cu") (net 18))
 (segment (start 136.258767 80.697233) (end 147.979767 80.697233) (width 0.2) (layer "F.Cu") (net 1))
 (segment (start 134.983767 81.972233) (end 136.258767 80.697233) (width 0.2) (layer "F.Cu") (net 1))
 (segment (start 132.998767 86.036233) (end 113.876767 86.036233) (width 0.2) (layer "F.Cu") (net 1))
 (segment (start 148.238767 80.956233) (end 148.238767 86.036233) (width 0.2) (layer "F.Cu") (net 1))
 (segment (start 113.876767 86.036233) (end 111.560767 88.352233) (width 0.2) (layer "F.Cu") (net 1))
 (segment (start 137.443767 118.548233) (end 140.110767 115.881233) (width 0.2) (layer "F.Cu") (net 1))
 (segment (start 140.110767 115.881233) (end 148.238767 115.881233) (width 0.2) (layer "F.Cu") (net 1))
 (segment (start 148.238767 119.691233) (end 148.238767 115.881233) (width 0.2) (layer "F.Cu") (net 1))
 (segment (start 148.238767 86.036233) (end 132.998767 86.036233) (width 0.2) (layer "F.Cu") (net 1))
 (segment (start 147.979767 80.697233) (end 148.238767 80.956233) (width 0.2) (layer "F.Cu") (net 1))
 (segment (start 148.238767 115.881233) (end 148.238767 86.036233) (width 0.2) (layer "F.Cu") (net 1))
 (segment (start 102.391767 118.548233) (end 102.391767 112.452233) (width 0.2) (layer "F.Cu") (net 20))
 (segment (start 102.391767 112.452233) (end 101.375767 111.436233) (width 0.2) (layer "F.Cu") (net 20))
 (via (at 101.375767 111.436233) (size 0.6) (drill 0.3) (layers "F.Cu" "B.Cu") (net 20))
 (segment (start 101.375767 110.587704) (end 100.250767 109.462704) (width 0.2) (layer "B.Cu") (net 20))
 (segment (start 100.250767 99.662233) (end 101.400767 98.512233) (width 0.2) (layer "B.Cu") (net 20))
 (segment (start 100.250767 109.462704) (end 100.250767 99.662233) (width 0.2) (layer "B.Cu") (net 20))
 (segment (start 101.375767 111.436233) (end 101.375767 110.587704) (width 0.2) (layer "B.Cu") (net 20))
 (segment (start 99.851767 118.548233) (end 99.851767 109.912233) (width 0.2) (layer "F.Cu") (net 19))
 (via (at 99.851767 109.912233) (size 0.6) (drill 0.3) (layers "F.Cu" "B.Cu") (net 19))
 (segment (start 97.819767 107.880233) (end 97.819767 99.553233) (width 0.2) (layer "B.Cu") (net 19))
 (segment (start 97.819767 99.553233) (end 101.400767 95.972233) (width 0.2) (layer "B.Cu") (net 19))
 (segment (start 99.851767 109.912233) (end 97.819767 107.880233) (width 0.2) (layer "B.Cu") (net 19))
 (segment (start 104.931767 104.583233) (end 101.400767 101.052233) (width 0.2) (layer "F.Cu") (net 21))
 (segment (start 104.931767 118.548233) (end 104.931767 104.583233) (width 0.2) (layer "F.Cu") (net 21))
 (segment (start 107.471767 118.548233) (end 107.471767 105.340233) (width 0.2) (layer "F.Cu") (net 9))
 (via (at 107.471767 105.340233) (size 0.6) (drill 0.3) (layers "F.Cu" "B.Cu") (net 9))
 (segment (start 107.471767 97.521233) (end 111.560767 93.432233) (width 0.2) (layer "B.Cu") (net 9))
 (segment (start 107.471767 105.340233) (end 107.471767 97.521233) (width 0.2) (layer "B.Cu") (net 9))
 (segment (start 112.551767 118.548233) (end 108.995767 114.992233) (width 0.2) (layer "F.Cu") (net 11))
 (segment (start 108.995767 114.484233) (end 108.995767 108.896233) (width 0.2) (layer "F.Cu") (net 11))
 (segment (start 108.995767 114.992233) (end 108.995767 114.484233) (width 0.2) (layer "F.Cu") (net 11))
 (via (at 108.995767 108.896233) (size 0.6) (drill 0.3) (layers "F.Cu" "B.Cu") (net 11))
 (segment (start 108.995767 101.077233) (end 111.560767 98.512233) (width 0.2) (layer "B.Cu") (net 11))
 (segment (start 108.995767 108.896233) (end 108.995767 101.077233) (width 0.2) (layer "B.Cu") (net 11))
 (segment (start 109.595767 113.052233) (end 109.595767 112.960233) (width 0.2) (layer "F.Cu") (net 12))
 (segment (start 115.091767 118.548233) (end 109.595767 113.052233) (width 0.2) (layer "F.Cu") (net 12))
 (via (at 109.595767 112.960233) (size 0.6) (drill 0.3) (layers "F.Cu" "B.Cu") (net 12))
 (segment (start 109.595767 112.960233) (end 109.595767 103.017233) (width 0.2) (layer "B.Cu") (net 12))
 (segment (start 109.595767 103.017233) (end 111.560767 101.052233) (width 0.2) (layer "B.Cu") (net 12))
 (segment (start 110.195767 111.112233) (end 110.195767 110.928233) (width 0.2) (layer "F.Cu") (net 13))
 (segment (start 117.631767 118.548233) (end 110.195767 111.112233) (width 0.2) (layer "F.Cu") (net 13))
 (via (at 110.195767 110.928233) (size 0.6) (drill 0.3) (layers "F.Cu" "B.Cu") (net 13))
 (segment (start 110.195767 104.957233) (end 111.560767 103.592233) (width 0.2) (layer "B.Cu") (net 13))
 (segment (start 110.195767 110.928233) (end 110.195767 104.957233) (width 0.2) (layer "B.Cu") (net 13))
 (segment (start 107.979767 112.036233) (end 108.071767 111.944233) (width 0.2) (layer "F.Cu") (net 10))
 (segment (start 110.011767 117.532233) (end 107.979767 115.500233) (width 0.2) (layer "F.Cu") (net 10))
 (segment (start 110.011767 118.548233) (end 110.011767 117.532233) (width 0.2) (layer "F.Cu") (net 10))
 (segment (start 107.979767 115.500233) (end 107.979767 112.036233) (width 0.2) (layer "F.Cu") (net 10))
 (via (at 108.071767 111.944233) (size 0.6) (drill 0.3) (layers "F.Cu" "B.Cu") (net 10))
 (segment (start 108.071767 111.944233) (end 108.071767 99.461233) (width 0.2) (layer "B.Cu") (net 10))
 (segment (start 108.071767 99.461233) (end 111.560767 95.972233) (width 0.2) (layer "B.Cu") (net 10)))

